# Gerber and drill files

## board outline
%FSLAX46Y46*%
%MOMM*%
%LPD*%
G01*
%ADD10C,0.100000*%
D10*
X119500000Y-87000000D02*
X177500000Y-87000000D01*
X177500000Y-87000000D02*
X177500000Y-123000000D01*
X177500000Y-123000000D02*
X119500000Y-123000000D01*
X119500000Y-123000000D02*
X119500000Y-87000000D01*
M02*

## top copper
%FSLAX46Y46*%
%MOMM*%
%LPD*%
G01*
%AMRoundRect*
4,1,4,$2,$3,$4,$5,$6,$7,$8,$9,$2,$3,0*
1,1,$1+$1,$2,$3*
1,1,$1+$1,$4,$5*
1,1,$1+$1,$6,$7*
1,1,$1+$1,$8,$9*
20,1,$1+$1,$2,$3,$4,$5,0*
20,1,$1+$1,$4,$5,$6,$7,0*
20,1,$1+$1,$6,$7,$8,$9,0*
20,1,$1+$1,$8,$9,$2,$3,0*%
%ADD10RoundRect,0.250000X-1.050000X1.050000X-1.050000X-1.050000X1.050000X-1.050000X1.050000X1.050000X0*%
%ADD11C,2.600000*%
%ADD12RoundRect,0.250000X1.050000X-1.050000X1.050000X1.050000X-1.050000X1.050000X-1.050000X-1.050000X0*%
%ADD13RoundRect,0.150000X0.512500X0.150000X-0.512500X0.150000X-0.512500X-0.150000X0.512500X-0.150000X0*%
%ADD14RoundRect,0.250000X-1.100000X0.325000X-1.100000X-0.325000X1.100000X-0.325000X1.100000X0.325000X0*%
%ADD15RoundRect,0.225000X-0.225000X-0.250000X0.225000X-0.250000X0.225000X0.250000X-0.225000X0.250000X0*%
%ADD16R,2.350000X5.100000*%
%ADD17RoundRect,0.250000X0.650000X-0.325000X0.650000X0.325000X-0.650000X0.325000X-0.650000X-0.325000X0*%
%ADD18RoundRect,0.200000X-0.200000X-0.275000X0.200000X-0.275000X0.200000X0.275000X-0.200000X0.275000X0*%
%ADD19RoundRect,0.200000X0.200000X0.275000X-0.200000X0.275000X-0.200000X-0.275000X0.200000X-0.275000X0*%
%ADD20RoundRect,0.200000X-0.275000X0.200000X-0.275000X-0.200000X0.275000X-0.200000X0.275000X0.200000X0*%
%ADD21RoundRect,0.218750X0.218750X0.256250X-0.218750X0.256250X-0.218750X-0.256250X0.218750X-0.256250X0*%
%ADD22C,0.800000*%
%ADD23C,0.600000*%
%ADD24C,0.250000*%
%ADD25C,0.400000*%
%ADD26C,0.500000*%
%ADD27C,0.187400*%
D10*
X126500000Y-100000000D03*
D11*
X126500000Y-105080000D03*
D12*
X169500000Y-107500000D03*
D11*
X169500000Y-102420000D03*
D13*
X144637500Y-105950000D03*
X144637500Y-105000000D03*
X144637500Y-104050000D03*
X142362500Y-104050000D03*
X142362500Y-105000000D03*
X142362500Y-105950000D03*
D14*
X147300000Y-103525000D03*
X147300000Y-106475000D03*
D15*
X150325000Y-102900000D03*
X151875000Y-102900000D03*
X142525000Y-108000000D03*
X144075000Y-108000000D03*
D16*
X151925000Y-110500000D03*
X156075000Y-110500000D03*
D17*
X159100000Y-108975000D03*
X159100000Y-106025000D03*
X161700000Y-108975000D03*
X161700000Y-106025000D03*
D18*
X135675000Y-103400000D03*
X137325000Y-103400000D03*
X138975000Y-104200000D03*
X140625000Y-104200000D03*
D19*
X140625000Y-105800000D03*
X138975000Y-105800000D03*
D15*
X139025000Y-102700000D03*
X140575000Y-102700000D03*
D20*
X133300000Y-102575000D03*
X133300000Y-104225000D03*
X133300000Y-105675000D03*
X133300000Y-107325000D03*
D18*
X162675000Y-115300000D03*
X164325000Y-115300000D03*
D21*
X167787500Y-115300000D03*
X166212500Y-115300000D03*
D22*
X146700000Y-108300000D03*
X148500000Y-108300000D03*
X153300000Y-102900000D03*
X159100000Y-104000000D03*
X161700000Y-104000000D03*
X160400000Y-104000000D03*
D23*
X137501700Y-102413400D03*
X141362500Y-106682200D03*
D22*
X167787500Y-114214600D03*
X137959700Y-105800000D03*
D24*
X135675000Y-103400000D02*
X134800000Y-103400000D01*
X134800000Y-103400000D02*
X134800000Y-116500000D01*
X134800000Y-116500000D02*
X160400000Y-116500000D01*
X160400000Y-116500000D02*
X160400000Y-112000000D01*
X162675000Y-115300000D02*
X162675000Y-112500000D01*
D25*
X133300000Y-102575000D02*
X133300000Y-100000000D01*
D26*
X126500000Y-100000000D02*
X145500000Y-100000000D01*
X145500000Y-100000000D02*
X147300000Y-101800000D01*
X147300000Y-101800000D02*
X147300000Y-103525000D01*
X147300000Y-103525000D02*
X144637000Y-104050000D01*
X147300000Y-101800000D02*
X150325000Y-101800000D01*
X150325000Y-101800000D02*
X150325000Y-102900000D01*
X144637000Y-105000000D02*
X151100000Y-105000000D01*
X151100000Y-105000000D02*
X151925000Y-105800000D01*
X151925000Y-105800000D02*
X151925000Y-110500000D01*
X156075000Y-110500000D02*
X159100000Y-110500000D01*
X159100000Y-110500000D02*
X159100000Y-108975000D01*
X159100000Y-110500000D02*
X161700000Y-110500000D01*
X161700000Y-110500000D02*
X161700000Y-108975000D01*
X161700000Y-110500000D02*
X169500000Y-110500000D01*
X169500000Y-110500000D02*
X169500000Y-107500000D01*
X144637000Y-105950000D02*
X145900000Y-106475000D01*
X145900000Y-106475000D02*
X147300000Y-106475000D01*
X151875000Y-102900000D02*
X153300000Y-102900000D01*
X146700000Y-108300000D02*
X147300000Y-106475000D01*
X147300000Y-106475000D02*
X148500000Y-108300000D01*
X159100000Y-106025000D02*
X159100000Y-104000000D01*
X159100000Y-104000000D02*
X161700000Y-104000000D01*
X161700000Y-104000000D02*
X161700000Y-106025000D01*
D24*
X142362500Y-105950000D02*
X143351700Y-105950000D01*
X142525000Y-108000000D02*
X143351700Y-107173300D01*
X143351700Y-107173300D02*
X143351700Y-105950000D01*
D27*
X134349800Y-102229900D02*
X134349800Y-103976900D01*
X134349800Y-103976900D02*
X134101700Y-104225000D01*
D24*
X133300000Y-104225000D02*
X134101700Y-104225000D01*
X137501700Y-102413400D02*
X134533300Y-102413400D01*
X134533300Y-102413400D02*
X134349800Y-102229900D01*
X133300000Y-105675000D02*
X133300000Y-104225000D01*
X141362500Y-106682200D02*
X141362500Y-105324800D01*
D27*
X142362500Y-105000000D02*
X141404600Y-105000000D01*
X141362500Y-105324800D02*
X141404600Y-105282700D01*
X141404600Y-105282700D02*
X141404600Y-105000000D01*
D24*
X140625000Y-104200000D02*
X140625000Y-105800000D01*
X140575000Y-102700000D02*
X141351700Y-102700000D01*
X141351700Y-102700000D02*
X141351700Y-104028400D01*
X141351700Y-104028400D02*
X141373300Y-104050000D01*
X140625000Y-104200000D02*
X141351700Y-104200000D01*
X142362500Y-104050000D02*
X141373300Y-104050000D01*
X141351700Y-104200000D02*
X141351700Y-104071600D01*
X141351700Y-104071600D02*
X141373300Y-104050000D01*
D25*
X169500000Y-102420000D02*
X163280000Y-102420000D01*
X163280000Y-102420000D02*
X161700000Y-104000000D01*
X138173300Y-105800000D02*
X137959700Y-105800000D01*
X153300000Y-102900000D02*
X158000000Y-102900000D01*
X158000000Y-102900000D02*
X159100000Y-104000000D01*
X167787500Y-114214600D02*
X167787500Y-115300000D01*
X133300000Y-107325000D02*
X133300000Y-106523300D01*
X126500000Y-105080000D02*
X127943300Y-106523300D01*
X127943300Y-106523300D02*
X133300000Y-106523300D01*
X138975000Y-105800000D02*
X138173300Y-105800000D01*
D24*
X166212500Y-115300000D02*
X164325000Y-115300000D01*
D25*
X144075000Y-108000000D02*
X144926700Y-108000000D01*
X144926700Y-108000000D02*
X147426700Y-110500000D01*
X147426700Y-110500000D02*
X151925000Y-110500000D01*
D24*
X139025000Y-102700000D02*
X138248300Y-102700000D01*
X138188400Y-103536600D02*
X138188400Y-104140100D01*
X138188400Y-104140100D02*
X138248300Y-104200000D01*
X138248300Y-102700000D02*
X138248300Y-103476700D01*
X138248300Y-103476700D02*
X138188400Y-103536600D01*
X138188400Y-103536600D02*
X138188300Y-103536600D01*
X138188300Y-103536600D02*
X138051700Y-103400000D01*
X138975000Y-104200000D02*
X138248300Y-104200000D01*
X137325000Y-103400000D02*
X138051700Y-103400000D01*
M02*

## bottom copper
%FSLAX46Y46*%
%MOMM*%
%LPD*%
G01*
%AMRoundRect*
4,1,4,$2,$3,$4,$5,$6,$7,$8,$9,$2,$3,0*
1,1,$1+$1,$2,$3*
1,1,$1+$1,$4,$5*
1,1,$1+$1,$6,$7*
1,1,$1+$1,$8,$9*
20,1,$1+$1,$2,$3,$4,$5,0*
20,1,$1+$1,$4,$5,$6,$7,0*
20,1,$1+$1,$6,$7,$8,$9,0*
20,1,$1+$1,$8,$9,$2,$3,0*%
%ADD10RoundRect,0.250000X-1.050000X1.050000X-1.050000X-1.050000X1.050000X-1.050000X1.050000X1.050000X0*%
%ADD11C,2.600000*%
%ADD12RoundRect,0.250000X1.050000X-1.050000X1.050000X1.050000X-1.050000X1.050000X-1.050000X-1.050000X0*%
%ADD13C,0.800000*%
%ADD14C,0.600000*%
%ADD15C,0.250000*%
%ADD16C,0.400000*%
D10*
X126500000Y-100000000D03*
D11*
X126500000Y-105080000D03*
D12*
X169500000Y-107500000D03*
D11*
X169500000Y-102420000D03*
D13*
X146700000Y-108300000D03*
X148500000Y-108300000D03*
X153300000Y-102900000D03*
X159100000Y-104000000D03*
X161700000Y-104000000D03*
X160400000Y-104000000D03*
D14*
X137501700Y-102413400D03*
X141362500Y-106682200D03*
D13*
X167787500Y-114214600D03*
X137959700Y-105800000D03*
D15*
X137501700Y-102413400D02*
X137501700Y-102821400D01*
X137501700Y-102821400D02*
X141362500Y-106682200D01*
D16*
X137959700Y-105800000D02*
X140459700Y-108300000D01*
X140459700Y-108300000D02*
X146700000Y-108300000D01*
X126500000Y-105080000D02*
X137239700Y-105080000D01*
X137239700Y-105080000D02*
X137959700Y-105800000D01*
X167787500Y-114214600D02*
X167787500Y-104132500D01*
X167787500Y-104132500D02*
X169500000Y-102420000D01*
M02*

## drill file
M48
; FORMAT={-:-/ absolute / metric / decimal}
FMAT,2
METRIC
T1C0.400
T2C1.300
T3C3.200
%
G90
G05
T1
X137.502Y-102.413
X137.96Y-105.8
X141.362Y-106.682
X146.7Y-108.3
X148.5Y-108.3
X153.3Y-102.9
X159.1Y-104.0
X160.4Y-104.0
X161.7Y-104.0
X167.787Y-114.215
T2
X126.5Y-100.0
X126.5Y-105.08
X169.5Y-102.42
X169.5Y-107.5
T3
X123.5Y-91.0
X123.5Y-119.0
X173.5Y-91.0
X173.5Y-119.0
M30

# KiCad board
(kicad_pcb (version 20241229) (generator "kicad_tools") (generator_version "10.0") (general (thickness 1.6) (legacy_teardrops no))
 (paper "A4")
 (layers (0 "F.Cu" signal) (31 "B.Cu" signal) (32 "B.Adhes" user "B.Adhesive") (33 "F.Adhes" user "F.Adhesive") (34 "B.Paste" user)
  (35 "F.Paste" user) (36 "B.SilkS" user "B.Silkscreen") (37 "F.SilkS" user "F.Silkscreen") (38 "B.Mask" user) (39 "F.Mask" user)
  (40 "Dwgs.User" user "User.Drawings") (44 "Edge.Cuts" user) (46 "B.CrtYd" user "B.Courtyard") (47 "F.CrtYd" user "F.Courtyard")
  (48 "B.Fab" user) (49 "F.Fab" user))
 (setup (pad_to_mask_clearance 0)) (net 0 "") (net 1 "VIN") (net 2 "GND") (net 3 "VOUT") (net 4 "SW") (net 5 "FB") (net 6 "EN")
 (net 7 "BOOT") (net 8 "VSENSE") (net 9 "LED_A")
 (gr_line (start 119.5 87) (end 177.5 87) (stroke (width 0.1) (type default)) (layer "Edge.Cuts"))
 (gr_line (start 177.5 87) (end 177.5 123) (stroke (width 0.1) (type default)) (layer "Edge.Cuts"))
 (gr_line (start 177.5 123) (end 119.5 123) (stroke (width 0.1) (type default)) (layer "Edge.Cuts"))
 (gr_line (start 119.5 123) (end 119.5 87) (stroke (width 0.1) (type default)) (layer "Edge.Cuts"))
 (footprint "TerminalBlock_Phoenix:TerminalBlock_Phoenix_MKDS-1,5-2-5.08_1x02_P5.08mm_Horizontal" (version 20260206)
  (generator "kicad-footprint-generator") (layer "F.Cu") (at 126.5 100 -90)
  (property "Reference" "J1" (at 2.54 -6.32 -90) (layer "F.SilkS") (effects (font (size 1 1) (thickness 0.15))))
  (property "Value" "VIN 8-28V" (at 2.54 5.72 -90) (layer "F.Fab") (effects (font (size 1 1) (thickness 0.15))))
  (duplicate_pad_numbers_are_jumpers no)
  (pad "1" thru_hole roundrect (at 0 0 -90) (size 2.6 2.6) (drill 1.3) (layers "*.Cu" "*.Mask") (remove_unused_layers no)
   (roundrect_rratio 0.096154) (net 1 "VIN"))
  (pad "2" thru_hole circle (at 5.08 0 -90) (size 2.6 2.6) (drill 1.3) (layers "*.Cu" "*.Mask") (remove_unused_layers no) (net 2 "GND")))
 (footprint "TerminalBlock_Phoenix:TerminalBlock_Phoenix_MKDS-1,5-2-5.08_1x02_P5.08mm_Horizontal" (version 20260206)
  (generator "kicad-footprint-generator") (layer "F.Cu") (at 169.5 107.5 90)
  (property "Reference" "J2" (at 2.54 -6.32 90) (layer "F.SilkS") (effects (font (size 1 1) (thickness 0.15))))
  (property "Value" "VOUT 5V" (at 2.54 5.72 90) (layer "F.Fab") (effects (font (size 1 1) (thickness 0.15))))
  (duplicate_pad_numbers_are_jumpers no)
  (pad "1" thru_hole roundrect (at 0 0 90) (size 2.6 2.6) (drill 1.3) (layers "*.Cu" "*.Mask") (remove_unused_layers no)
   (roundrect_rratio 0.096154) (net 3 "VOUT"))
  (pad "2" thru_hole circle (at 5.08 0 90) (size 2.6 2.6) (drill 1.3) (layers "*.Cu" "*.Mask") (remove_unused_layers no) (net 2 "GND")))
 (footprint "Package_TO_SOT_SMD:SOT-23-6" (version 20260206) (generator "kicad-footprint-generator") (layer "F.Cu") (at 143.5 105 180)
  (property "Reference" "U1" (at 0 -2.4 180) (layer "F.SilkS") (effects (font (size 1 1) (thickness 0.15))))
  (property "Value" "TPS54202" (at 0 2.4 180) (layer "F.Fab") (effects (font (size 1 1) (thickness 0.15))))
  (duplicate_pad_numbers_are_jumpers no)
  (pad "1" smd roundrect (at -1.1375 -0.95 180) (size 1.325 0.6) (layers "F.Cu" "F.Mask" "F.Paste") (roundrect_rratio 0.25) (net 2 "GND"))
  (pad "2" smd roundrect (at -1.1375 0 180) (size 1.325 0.6) (layers "F.Cu" "F.Mask" "F.Paste") (roundrect_rratio 0.25) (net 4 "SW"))
  (pad "3" smd roundrect (at -1.1375 0.95 180) (size 1.325 0.6) (layers "F.Cu" "F.Mask" "F.Paste") (roundrect_rratio 0.25) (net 1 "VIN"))
  (pad "4" smd roundrect (at 1.1375 0.95 180) (size 1.325 0.6) (layers "F.Cu" "F.Mask" "F.Paste") (roundrect_rratio 0.25) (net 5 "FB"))
  (pad "5" smd roundrect (at 1.1375 0 180) (size 1.325 0.6) (layers "F.Cu" "F.Mask" "F.Paste") (roundrect_rratio 0.25) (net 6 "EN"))
  (pad "6" smd roundrect (at 1.1375 -0.95 180) (size 1.325 0.6) (layers "F.Cu" "F.Mask" "F.Paste") (roundrect_rratio 0.25) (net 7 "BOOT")))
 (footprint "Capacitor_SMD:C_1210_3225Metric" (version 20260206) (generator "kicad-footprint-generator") (layer "F.Cu") (at 147.3 105 -90)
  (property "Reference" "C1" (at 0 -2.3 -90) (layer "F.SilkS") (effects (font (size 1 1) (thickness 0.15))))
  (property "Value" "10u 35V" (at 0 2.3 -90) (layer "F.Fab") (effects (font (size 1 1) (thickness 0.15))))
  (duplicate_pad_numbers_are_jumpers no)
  (pad "1" smd roundrect (at -1.475 0 -90) (size 1.15 2.7) (layers "F.Cu" "F.Mask" "F.Paste") (roundrect_rratio 0.217391) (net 1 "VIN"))
  (pad "2" smd roundrect (at 1.475 0 -90) (size 1.15 2.7) (layers "F.Cu" "F.Mask" "F.Paste") (roundrect_rratio 0.217391) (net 2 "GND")))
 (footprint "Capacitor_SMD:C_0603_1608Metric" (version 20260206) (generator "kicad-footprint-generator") (layer "F.Cu") (at 151.1 102.9)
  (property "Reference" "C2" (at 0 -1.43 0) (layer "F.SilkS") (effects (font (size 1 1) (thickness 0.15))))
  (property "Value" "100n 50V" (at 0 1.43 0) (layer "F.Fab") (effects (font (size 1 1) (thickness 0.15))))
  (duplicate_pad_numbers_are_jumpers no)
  (pad "1" smd roundrect (at -0.775 0) (size 0.9 0.95) (layers "F.Cu" "F.Mask" "F.Paste") (roundrect_rratio 0.25) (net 1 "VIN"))
  (pad "2" smd roundrect (at 0.775 0) (size 0.9 0.95) (layers "F.Cu" "F.Mask" "F.Paste") (roundrect_rratio 0.25) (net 2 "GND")))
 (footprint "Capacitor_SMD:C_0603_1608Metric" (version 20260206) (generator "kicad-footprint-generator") (layer "F.Cu") (at 143.3 108)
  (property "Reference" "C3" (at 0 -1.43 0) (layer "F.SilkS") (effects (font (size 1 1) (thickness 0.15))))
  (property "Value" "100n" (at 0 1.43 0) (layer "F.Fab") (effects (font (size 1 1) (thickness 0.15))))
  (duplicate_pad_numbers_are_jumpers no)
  (pad "1" smd roundrect (at -0.775 0) (size 0.9 0.95) (layers "F.Cu" "F.Mask" "F.Paste") (roundrect_rratio 0.25) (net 7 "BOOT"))
  (pad "2" smd roundrect (at 0.775 0) (size 0.9 0.95) (layers "F.Cu" "F.Mask" "F.Paste") (roundrect_rratio 0.25) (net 4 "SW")))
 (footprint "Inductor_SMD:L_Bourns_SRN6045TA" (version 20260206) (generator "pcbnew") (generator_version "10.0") (layer "F.Cu")
  (at 154 110.5)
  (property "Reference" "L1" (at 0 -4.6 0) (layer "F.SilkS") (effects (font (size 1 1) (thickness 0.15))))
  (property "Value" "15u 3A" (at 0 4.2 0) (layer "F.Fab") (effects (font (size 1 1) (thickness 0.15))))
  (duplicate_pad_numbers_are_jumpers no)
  (pad "1" smd rect (at -2.075 0) (size 2.35 5.1) (layers "F.Cu" "F.Mask" "F.Paste") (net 4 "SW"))
  (pad "2" smd rect (at 2.075 0) (size 2.35 5.1) (layers "F.Cu" "F.Mask" "F.Paste") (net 3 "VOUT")))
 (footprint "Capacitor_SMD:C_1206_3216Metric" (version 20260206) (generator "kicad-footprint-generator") (layer "F.Cu") (at 159.1 107.5 90)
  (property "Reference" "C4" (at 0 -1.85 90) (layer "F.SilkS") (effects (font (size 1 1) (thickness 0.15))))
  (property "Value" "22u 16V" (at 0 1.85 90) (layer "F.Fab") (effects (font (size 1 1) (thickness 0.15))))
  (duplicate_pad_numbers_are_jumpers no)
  (pad "1" smd roundrect (at -1.475 0 90) (size 1.15 1.8) (layers "F.Cu" "F.Mask" "F.Paste") (roundrect_rratio 0.217391) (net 3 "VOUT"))
  (pad "2" smd roundrect (at 1.475 0 90) (size 1.15 1.8) (layers "F.Cu" "F.Mask" "F.Paste") (roundrect_rratio 0.217391) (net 2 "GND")))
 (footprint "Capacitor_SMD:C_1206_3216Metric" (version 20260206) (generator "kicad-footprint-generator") (layer "F.Cu") (at 161.7 107.5 90)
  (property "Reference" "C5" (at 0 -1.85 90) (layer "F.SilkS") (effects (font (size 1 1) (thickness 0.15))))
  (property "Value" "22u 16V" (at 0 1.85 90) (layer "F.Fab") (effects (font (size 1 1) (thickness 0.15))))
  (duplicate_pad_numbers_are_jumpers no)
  (pad "1" smd roundrect (at -1.475 0 90) (size 1.15 1.8) (layers "F.Cu" "F.Mask" "F.Paste") (roundrect_rratio 0.217391) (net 3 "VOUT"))
  (pad "2" smd roundrect (at 1.475 0 90) (size 1.15 1.8) (layers "F.Cu" "F.Mask" "F.Paste") (roundrect_rratio 0.217391) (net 2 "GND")))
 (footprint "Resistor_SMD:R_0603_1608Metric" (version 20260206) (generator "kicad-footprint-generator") (layer "F.Cu") (at 136.5 103.4)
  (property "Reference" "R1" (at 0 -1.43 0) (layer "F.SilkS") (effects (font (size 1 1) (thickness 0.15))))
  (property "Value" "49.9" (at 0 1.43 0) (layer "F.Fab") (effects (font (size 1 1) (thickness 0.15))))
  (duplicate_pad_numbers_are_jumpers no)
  (pad "1" smd roundrect (at -0.825 0) (size 0.8 0.95) (layers "F.Cu" "F.Mask" "F.Paste") (roundrect_rratio 0.25) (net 3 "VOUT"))
  (pad "2" smd roundrect (at 0.825 0) (size 0.8 0.95) (layers "F.Cu" "F.Mask" "F.Paste") (roundrect_rratio 0.25) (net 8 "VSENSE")))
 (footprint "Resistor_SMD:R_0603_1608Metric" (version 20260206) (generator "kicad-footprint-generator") (layer "F.Cu") (at 139.8 104.2)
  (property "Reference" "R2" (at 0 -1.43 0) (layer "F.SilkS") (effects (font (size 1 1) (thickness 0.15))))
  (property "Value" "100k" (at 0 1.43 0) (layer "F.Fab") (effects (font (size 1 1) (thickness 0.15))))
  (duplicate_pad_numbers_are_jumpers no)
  (pad "1" smd roundrect (at -0.825 0) (size 0.8 0.95) (layers "F.Cu" "F.Mask" "F.Paste") (roundrect_rratio 0.25) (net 8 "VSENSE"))
  (pad "2" smd roundrect (at 0.825 0) (size 0.8 0.95) (layers "F.Cu" "F.Mask" "F.Paste") (roundrect_rratio 0.25) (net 5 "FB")))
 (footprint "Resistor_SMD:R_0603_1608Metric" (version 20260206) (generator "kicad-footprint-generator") (layer "F.Cu") (at 139.8 105.8 180)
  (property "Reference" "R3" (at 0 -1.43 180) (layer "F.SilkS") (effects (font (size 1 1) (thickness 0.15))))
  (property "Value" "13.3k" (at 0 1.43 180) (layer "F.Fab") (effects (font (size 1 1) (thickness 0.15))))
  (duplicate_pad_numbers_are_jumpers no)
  (pad "1" smd roundrect (at -0.825 0 180) (size 0.8 0.95) (layers "F.Cu" "F.Mask" "F.Paste") (roundrect_rratio 0.25) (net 5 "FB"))
  (pad "2" smd roundrect (at 0.825 0 180) (size 0.8 0.95) (layers "F.Cu" "F.Mask" "F.Paste") (roundrect_rratio 0.25) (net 2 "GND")))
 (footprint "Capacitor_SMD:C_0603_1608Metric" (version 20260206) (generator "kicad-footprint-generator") (layer "F.Cu") (at 139.8 102.7)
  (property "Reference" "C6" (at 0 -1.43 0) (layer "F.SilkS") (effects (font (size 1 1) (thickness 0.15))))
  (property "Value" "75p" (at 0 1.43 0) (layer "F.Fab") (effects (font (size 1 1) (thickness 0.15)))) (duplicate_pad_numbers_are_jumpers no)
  (pad "1" smd roundrect (at -0.775 0) (size 0.9 0.95) (layers "F.Cu" "F.Mask" "F.Paste") (roundrect_rratio 0.25) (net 8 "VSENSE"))
  (pad "2" smd roundrect (at 0.775 0) (size 0.9 0.95) (layers "F.Cu" "F.Mask" "F.Paste") (roundrect_rratio 0.25) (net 5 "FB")))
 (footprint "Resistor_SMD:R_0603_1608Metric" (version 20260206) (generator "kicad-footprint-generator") (layer "F.Cu") (at 133.3 103.4 -90)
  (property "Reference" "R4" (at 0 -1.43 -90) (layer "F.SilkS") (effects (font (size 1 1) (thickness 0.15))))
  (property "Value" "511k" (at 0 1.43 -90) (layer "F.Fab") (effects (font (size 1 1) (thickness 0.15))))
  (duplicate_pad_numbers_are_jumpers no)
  (pad "1" smd roundrect (at -0.825 0 -90) (size 0.8 0.95) (layers "F.Cu" "F.Mask" "F.Paste") (roundrect_rratio 0.25) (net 1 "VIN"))
  (pad "2" smd roundrect (at 0.825 0 -90) (size 0.8 0.95) (layers "F.Cu" "F.Mask" "F.Paste") (roundrect_rratio 0.25) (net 6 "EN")))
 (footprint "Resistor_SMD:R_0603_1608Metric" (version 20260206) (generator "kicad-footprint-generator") (layer "F.Cu") (at 133.3 106.5 -90)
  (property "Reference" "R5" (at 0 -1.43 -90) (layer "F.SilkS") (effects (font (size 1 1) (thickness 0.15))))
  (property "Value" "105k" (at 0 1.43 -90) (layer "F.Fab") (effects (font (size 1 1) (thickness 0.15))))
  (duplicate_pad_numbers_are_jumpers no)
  (pad "1" smd roundrect (at -0.825 0 -90) (size 0.8 0.95) (layers "F.Cu" "F.Mask" "F.Paste") (roundrect_rratio 0.25) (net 6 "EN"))
  (pad "2" smd roundrect (at 0.825 0 -90) (size 0.8 0.95) (layers "F.Cu" "F.Mask" "F.Paste") (roundrect_rratio 0.25) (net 2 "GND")))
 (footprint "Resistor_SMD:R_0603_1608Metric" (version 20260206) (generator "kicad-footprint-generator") (layer "F.Cu") (at 163.5 115.3)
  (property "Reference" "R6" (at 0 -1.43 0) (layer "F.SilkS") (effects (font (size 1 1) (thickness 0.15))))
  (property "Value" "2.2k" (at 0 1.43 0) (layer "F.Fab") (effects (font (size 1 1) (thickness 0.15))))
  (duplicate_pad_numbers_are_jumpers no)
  (pad "1" smd roundrect (at -0.825 0) (size 0.8 0.95) (layers "F.Cu" "F.Mask" "F.Paste") (roundrect_rratio 0.25) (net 3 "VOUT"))
  (pad "2" smd roundrect (at 0.825 0) (size 0.8 0.95) (layers "F.Cu" "F.Mask" "F.Paste") (roundrect_rratio 0.25) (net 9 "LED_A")))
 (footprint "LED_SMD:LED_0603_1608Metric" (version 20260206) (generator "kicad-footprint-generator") (layer "F.Cu") (at 167 115.3 180)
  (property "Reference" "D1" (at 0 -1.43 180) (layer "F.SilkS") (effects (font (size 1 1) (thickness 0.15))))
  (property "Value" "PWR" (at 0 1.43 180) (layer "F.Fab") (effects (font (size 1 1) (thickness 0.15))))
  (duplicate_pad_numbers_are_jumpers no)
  (pad "1" smd roundrect (at -0.7875 0 180) (size 0.875 0.95) (layers "F.Cu" "F.Mask" "F.Paste") (roundrect_rratio 0.25) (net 2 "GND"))
  (pad "2" smd roundrect (at 0.7875 0 180) (size 0.875 0.95) (layers "F.Cu" "F.Mask" "F.Paste") (roundrect_rratio 0.25) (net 9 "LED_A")))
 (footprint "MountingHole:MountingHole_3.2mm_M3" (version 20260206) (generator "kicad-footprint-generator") (layer "F.Cu") (at 123.5 91)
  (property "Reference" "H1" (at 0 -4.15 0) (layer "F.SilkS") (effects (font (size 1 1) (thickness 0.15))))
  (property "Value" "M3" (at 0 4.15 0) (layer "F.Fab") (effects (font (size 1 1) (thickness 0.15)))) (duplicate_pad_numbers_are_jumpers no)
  (pad "" np_thru_hole circle (at 0 0) (size 3.2 3.2) (drill 3.2) (layers "*.Cu" "*.Mask")))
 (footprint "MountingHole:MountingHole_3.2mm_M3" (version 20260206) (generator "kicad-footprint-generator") (layer "F.Cu") (at 173.5 91)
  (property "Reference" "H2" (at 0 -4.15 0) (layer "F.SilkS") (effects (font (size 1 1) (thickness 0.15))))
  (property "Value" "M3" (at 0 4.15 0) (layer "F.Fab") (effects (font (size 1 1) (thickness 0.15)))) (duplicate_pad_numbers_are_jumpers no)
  (pad "" np_thru_hole circle (at 0 0) (size 3.2 3.2) (drill 3.2) (layers "*.Cu" "*.Mask")))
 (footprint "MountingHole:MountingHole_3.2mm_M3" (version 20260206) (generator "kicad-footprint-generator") (layer "F.Cu") (at 123.5 119)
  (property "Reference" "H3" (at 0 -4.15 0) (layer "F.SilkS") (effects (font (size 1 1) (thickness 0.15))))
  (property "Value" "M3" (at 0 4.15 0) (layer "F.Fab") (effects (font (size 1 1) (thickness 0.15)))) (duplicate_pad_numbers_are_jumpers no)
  (pad "" np_thru_hole circle (at 0 0) (size 3.2 3.2) (drill 3.2) (layers "*.Cu" "*.Mask")))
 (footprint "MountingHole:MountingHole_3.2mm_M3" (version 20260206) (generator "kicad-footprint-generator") (layer "F.Cu") (at 173.5 119)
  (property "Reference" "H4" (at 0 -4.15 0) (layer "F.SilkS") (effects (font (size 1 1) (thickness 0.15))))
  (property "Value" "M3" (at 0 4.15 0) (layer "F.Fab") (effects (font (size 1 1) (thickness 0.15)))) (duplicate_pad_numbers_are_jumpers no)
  (pad "" np_thru_hole circle (at 0 0) (size 3.2 3.2) (drill 3.2) (layers "*.Cu" "*.Mask")))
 (via (at 146.7 108.3) (size 0.8) (drill 0.4) (layers "F.Cu" "B.Cu") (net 2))
 (via (at 148.5 108.3) (size 0.8) (drill 0.4) (layers "F.Cu" "B.Cu") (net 2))
 (via (at 153.3 102.9) (size 0.8) (drill 0.4) (layers "F.Cu" "B.Cu") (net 2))
 (via (at 159.1 104.0) (size 0.8) (drill 0.4) (layers "F.Cu" "B.Cu") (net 2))
 (via (at 161.7 104.0) (size 0.8) (drill 0.4) (layers "F.Cu" "B.Cu") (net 2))
 (via (at 160.4 104.0) (size 0.8) (drill 0.4) (layers "F.Cu" "B.Cu") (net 2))
 (segment (start 135.675 103.4) (end 134.8 103.4) (width 0.25) (layer "F.Cu") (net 3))
 (segment (start 134.8 103.4) (end 134.8 116.5) (width 0.25) (layer "F.Cu") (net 3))
 (segment (start 134.8 116.5) (end 160.4 116.5) (width 0.25) (layer "F.Cu") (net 3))
 (segment (start 160.4 116.5) (end 160.4 112.0) (width 0.25) (layer "F.Cu") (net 3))
 (segment (start 162.675 115.3) (end 162.675 112.5) (width 0.25) (layer "F.Cu") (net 3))
 (segment (start 133.3 102.575) (end 133.3 100.0) (width 0.4) (layer "F.Cu") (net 1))
 (segment (start 126.5 100.0) (end 145.5 100.0) (width 0.5) (layer "F.Cu") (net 1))
 (segment (start 145.5 100.0) (end 147.3 101.8) (width 0.5) (layer "F.Cu") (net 1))
 (segment (start 147.3 101.8) (end 147.3 103.525) (width 0.5) (layer "F.Cu") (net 1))
 (segment (start 147.3 103.525) (end 144.637 104.05) (width 0.5) (layer "F.Cu") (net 1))
 (segment (start 147.3 101.8) (end 150.325 101.8) (width 0.5) (layer "F.Cu") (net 1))
 (segment (start 150.325 101.8) (end 150.325 102.9) (width 0.5) (layer "F.Cu") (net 1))
 (segment (start 144.637 105.0) (end 151.1 105.0) (width 0.5) (layer "F.Cu") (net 4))
 (segment (start 151.1 105.0) (end 151.925 105.8) (width 0.5) (layer "F.Cu") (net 4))
 (segment (start 151.925 105.8) (end 151.925 110.5) (width 0.5) (layer "F.Cu") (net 4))
 (segment (start 156.075 110.5) (end 159.1 110.5) (width 0.5) (layer "F.Cu") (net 3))
 (segment (start 159.1 110.5) (end 159.1 108.975) (width 0.5) (layer "F.Cu") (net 3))
 (segment (start 159.1 110.5) (end 161.7 110.5) (width 0.5) (layer "F.Cu") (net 3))
 (segment (start 161.7 110.5) (end 161.7 108.975) (width 0.5) (layer "F.Cu") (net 3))
 (segment (start 161.7 110.5) (end 169.5 110.5) (width 0.5) (layer "F.Cu") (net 3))
 (segment (start 169.5 110.5) (end 169.5 107.5) (width 0.5) (layer "F.Cu") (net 3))
 (segment (start 144.637 105.95) (end 145.9 106.475) (width 0.5) (layer "F.Cu") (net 2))
 (segment (start 145.9 106.475) (end 147.3 106.475) (width 0.5) (layer "F.Cu") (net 2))
 (segment (start 151.875 102.9) (end 153.3 102.9) (width 0.5) (layer "F.Cu") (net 2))
 (segment (start 146.7 108.3) (end 147.3 106.475) (width 0.5) (layer "F.Cu") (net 2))
 (segment (start 147.3 106.475) (end 148.5 108.3) (width 0.5) (layer "F.Cu") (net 2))
 (segment (start 159.1 106.025) (end 159.1 104.0) (width 0.5) (layer "F.Cu") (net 2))
 (segment (start 159.1 104.0) (end 161.7 104.0) (width 0.5) (layer "F.Cu") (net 2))
 (segment (start 161.7 104.0) (end 161.7 106.025) (width 0.5) (layer "F.Cu") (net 2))
 (segment (start 142.3625 105.9500) (end 143.3517 105.9500) (width 0.2500) (layer "F.Cu") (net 7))
 (segment (start 142.5250 108.0000) (end 143.3517 107.1733) (width 0.2500) (layer "F.Cu") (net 7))
 (segment (start 143.3517 107.1733) (end 143.3517 105.9500) (width 0.2500) (layer "F.Cu") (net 7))
 (segment (start 137.5017 102.4134) (end 137.5017 102.8214) (width 0.2500) (layer "B.Cu") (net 6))
 (segment (start 137.5017 102.8214) (end 141.3625 106.6822) (width 0.2500) (layer "B.Cu") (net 6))
 (segment (start 134.3498 102.2299) (end 134.3498 103.9769) (width 0.1874) (layer "F.Cu") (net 6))
 (segment (start 134.3498 103.9769) (end 134.1017 104.2250) (width 0.1874) (layer "F.Cu") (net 6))
 (segment (start 133.3000 104.2250) (end 134.1017 104.2250) (width 0.2500) (layer "F.Cu") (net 6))
 (segment (start 137.5017 102.4134) (end 134.5333 102.4134) (width 0.2500) (layer "F.Cu") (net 6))
 (segment (start 134.5333 102.4134) (end 134.3498 102.2299) (width 0.2500) (layer "F.Cu") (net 6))
 (segment (start 133.3000 105.6750) (end 133.3000 104.2250) (width 0.2500) (layer "F.Cu") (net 6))
 (segment (start 141.3625 106.6822) (end 141.3625 105.3248) (width 0.2500) (layer "F.Cu") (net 6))
 (segment (start 142.3625 105.0000) (end 141.4046 105.0000) (width 0.1874) (layer "F.Cu") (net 6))
 (segment (start 141.3625 105.3248) (end 141.4046 105.2827) (width 0.1874) (layer "F.Cu") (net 6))
 (segment (start 141.4046 105.2827) (end 141.4046 105.0000) (width 0.1874) (layer "F.Cu") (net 6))
 (segment (start 140.6250 104.2000) (end 140.6250 105.8000) (width 0.2500) (layer "F.Cu") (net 5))
 (segment (start 140.5750 102.7000) (end 141.3517 102.7000) (width 0.2500) (layer "F.Cu") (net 5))
 (segment (start 141.3517 102.7000) (end 141.3517 104.0284) (width 0.2500) (layer "F.Cu") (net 5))
 (segment (start 141.3517 104.0284) (end 141.3733 104.0500) (width 0.2500) (layer "F.Cu") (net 5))
 (segment (start 140.6250 104.2000) (end 141.3517 104.2000) (width 0.2500) (layer "F.Cu") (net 5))
 (segment (start 142.3625 104.0500) (end 141.3733 104.0500) (width 0.2500) (layer "F.Cu") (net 5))
 (segment (start 141.3517 104.2000) (end 141.3517 104.0716) (width 0.2500) (layer "F.Cu") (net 5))
 (segment (start 141.3517 104.0716) (end 141.3733 104.0500) (width 0.2500) (layer "F.Cu") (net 5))
 (segment (start 169.5000 102.4200) (end 163.2800 102.4200) (width 0.4000) (layer "F.Cu") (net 2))
 (segment (start 163.2800 102.4200) (end 161.7000 104.0000) (width 0.4000) (layer "F.Cu") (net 2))
 (segment (start 137.9597 105.8000) (end 140.4597 108.3000) (width 0.4000) (layer "B.Cu") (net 2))
 (segment (start 140.4597 108.3000) (end 146.7000 108.3000) (width 0.4000) (layer "B.Cu") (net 2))
 (segment (start 138.1733 105.8000) (end 137.9597 105.8000) (width 0.4000) (layer "F.Cu") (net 2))
 (segment (start 126.5000 105.0800) (end 137.2397 105.0800) (width 0.4000) (layer "B.Cu") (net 2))
 (segment (start 137.2397 105.0800) (end 137.9597 105.8000) (width 0.4000) (layer "B.Cu") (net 2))
 (segment (start 167.7875 114.2146) (end 167.7875 104.1325) (width 0.4000) (layer "B.Cu") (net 2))
 (segment (start 167.7875 104.1325) (end 169.5000 102.4200) (width 0.4000) (layer "B.Cu") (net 2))
 (segment (start 153.3000 102.9000) (end 158.0000 102.9000) (width 0.4000) (layer "F.Cu") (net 2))
 (segment (start 158.0000 102.9000) (end 159.1000 104.0000) (width 0.4000) (layer "F.Cu") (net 2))
 (segment (start 167.7875 114.2146) (end 167.7875 115.3000) (width 0.4000) (layer "F.Cu") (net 2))
 (segment (start 133.3000 107.3250) (end 133.3000 106.5233) (width 0.4000) (layer "F.Cu") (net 2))
 (segment (start 126.5000 105.0800) (end 127.9433 106.5233) (width 0.4000) (layer "F.Cu") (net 2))
 (segment (start 127.9433 106.5233) (end 133.3000 106.5233) (width 0.4000) (layer "F.Cu") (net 2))
 (segment (start 138.9750 105.8000) (end 138.1733 105.8000) (width 0.4000) (layer "F.Cu") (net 2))
 (segment (start 166.2125 115.3000) (end 164.3250 115.3000) (width 0.2500) (layer "F.Cu") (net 9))
 (segment (start 144.0750 108.0000) (end 144.9267 108.0000) (width 0.4000) (layer "F.Cu") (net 4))
 (segment (start 144.9267 108.0000) (end 147.4267 110.5000) (width 0.4000) (layer "F.Cu") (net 4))
 (segment (start 147.4267 110.5000) (end 151.9250 110.5000) (width 0.4000) (layer "F.Cu") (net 4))
 (segment (start 139.0250 102.7000) (end 138.2483 102.7000) (width 0.2500) (layer "F.Cu") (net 8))
 (segment (start 138.1884 103.5366) (end 138.1884 104.1401) (width 0.2500) (layer "F.Cu") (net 8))
 (segment (start 138.1884 104.1401) (end 138.2483 104.2000) (width 0.2500) (layer "F.Cu") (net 8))
 (segment (start 138.2483 102.7000) (end 138.2483 103.4767) (width 0.2500) (layer "F.Cu") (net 8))
 (segment (start 138.2483 103.4767) (end 138.1884 103.5366) (width 0.2500) (layer "F.Cu") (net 8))
 (segment (start 138.1884 103.5366) (end 138.1883 103.5366) (width 0.2500) (layer "F.Cu") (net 8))
 (segment (start 138.1883 103.5366) (end 138.0517 103.4000) (width 0.2500) (layer "F.Cu") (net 8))
 (segment (start 138.9750 104.2000) (end 138.2483 104.2000) (width 0.2500) (layer "F.Cu") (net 8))
 (segment (start 137.3250 103.4000) (end 138.0517 103.4000) (width 0.2500) (layer "F.Cu") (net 8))
 (via (at 137.5017 102.4134) (size 0.6000) (drill 0.4) (layers "F.Cu" "B.Cu") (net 6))
 (via (at 141.3625 106.6822) (size 0.6000) (drill 0.4) (layers "F.Cu" "B.Cu") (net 6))
 (via (at 167.7875 114.2146) (size 0.8000) (drill 0.4) (layers "F.Cu" "B.Cu") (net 2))
 (via (at 137.9597 105.8000) (size 0.8000) (drill 0.4) (layers "F.Cu" "B.Cu") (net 2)))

